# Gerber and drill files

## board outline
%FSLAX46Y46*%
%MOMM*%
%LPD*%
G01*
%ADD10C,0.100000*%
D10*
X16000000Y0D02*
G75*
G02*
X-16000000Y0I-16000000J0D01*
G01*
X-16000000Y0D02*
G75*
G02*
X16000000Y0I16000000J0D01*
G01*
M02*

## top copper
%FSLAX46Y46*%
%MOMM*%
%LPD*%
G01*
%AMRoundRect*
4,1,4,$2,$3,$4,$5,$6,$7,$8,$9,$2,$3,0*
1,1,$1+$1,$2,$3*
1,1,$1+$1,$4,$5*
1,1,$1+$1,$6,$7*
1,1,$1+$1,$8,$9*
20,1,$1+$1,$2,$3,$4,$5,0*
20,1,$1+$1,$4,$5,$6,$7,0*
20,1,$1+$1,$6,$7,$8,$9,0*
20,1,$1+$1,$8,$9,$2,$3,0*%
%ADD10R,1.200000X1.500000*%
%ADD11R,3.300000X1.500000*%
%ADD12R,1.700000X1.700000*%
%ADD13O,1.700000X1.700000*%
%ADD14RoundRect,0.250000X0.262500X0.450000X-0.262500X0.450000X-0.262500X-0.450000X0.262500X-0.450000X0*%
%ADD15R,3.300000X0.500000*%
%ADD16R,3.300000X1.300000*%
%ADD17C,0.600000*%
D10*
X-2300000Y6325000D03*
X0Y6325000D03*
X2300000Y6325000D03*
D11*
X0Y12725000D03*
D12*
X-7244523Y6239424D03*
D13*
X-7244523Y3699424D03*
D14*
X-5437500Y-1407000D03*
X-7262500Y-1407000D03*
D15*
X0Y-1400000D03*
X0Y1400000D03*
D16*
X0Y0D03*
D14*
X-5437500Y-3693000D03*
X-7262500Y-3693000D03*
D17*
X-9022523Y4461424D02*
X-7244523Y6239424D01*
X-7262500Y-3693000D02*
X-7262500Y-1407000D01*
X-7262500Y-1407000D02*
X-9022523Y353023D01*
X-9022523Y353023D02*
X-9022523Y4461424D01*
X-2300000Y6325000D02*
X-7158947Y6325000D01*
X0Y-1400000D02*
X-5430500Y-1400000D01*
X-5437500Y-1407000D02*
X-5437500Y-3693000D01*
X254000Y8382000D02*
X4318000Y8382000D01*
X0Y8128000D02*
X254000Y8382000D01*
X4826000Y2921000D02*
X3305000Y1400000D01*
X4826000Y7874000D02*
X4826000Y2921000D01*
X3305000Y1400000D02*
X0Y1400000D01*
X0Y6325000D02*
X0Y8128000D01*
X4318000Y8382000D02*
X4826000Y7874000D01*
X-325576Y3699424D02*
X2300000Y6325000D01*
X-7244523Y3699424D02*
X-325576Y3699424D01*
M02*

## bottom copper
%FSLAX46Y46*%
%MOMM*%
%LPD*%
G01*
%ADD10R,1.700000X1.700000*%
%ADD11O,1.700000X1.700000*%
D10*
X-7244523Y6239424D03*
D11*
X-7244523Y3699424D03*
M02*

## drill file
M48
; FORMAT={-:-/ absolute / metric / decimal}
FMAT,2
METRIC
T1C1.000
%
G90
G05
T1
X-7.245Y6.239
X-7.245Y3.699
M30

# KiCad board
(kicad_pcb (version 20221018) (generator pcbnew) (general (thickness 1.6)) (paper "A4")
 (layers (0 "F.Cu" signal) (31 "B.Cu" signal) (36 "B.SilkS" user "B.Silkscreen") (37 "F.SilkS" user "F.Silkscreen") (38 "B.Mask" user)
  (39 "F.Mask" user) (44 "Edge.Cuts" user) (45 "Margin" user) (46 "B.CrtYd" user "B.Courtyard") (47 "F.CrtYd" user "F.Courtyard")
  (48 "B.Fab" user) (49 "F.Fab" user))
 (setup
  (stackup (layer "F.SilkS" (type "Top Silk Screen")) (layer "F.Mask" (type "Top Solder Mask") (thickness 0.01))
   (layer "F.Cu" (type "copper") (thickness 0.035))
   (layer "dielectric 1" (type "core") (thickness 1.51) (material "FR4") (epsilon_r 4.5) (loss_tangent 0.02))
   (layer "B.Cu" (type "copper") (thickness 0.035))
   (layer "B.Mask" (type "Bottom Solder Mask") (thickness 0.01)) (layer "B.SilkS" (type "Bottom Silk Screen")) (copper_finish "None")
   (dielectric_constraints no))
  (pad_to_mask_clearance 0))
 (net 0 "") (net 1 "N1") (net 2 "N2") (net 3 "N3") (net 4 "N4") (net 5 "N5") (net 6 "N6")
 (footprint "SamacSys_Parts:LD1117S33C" (layer "F.Cu") (at 0 -9.525)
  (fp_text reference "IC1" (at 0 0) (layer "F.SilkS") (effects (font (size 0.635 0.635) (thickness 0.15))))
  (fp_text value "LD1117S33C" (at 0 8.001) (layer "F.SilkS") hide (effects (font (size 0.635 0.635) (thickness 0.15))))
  (pad "1" smd rect (at -2.3 3.2) (size 1.2 1.5) (layers "F.Cu" "F.Paste" "F.Mask") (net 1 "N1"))
  (pad "2" smd rect (at 0 3.2) (size 1.2 1.5) (layers "F.Cu" "F.Paste" "F.Mask") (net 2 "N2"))
  (pad "3" smd rect (at 2.3 3.2) (size 1.2 1.5) (layers "F.Cu" "F.Paste" "F.Mask") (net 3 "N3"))
  (pad "4" smd rect (at 0 -3.2 90) (size 1.5 3.3) (layers "F.Cu" "F.Paste" "F.Mask") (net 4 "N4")))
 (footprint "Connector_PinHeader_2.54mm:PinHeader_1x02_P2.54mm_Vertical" (layer "F.Cu") (at -7.244523 -6.239424)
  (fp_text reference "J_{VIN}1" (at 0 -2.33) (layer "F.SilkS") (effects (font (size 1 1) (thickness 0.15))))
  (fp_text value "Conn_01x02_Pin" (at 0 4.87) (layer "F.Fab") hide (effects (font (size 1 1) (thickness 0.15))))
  (pad "1" thru_hole rect (at 0 0) (size 1.7 1.7) (drill 1) (layers "*.Cu" "*.Mask") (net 1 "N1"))
  (pad "2" thru_hole oval (at 0 2.54) (size 1.7 1.7) (drill 1) (layers "*.Cu" "*.Mask") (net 3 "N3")))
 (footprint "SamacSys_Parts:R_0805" (layer "F.Cu") (at -6.35 1.397 90)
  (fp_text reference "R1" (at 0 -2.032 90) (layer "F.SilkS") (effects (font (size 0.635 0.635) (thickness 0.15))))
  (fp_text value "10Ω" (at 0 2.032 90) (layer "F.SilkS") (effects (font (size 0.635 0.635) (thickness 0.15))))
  (pad "1" smd roundrect (at -0.01 0.9125 180) (size 1.025 1.4) (layers "F.Cu" "F.Paste" "F.Mask") (roundrect_rratio 0.243902439)
   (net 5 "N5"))
  (pad "2" smd roundrect (at -0.01 -0.9125 180) (size 1.025 1.4) (layers "F.Cu" "F.Paste" "F.Mask") (roundrect_rratio 0.243902439)
   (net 1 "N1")))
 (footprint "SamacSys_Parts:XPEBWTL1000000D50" (layer "F.Cu") (at 0 0 90)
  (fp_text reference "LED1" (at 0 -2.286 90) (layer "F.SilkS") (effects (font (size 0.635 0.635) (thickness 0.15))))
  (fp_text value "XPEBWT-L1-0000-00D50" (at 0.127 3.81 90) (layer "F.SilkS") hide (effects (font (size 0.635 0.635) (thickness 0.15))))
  (pad "1" smd rect (at -1.4 0 90) (size 0.5 3.3) (layers "F.Cu" "F.Paste" "F.Mask") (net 5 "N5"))
  (pad "2" smd rect (at 1.4 0 90) (size 0.5 3.3) (layers "F.Cu" "F.Paste" "F.Mask") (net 2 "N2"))
  (pad "3" smd rect (at 0 0 90) (size 1.3 3.3) (layers "F.Cu" "F.Paste" "F.Mask") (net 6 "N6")))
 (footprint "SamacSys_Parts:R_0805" (layer "F.Cu") (at -6.35 3.683 90)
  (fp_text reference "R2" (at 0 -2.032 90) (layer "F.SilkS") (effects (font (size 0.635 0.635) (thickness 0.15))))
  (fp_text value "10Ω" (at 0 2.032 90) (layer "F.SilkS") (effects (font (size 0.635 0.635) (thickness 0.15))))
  (pad "1" smd roundrect (at -0.01 0.9125 180) (size 1.025 1.4) (layers "F.Cu" "F.Paste" "F.Mask") (roundrect_rratio 0.243902439)
   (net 5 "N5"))
  (pad "2" smd roundrect (at -0.01 -0.9125 180) (size 1.025 1.4) (layers "F.Cu" "F.Paste" "F.Mask") (roundrect_rratio 0.243902439)
   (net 1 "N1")))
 (gr_circle (center 0 0) (end 16 0) (stroke (width 0.1) (type default)) (fill none) (layer "Edge.Cuts"))
 (segment (start -9.022523 -4.461424) (end -7.244523 -6.239424) (width 0.6) (layer "F.Cu") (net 1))
 (segment (start -7.2625 3.693) (end -7.2625 1.407) (width 0.6) (layer "F.Cu") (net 1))
 (segment (start -7.2625 1.407) (end -9.022523 -0.353023) (width 0.6) (layer "F.Cu") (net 1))
 (segment (start -9.022523 -0.353023) (end -9.022523 -4.461424) (width 0.6) (layer "F.Cu") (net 1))
 (segment (start -2.3 -6.325) (end -7.158947 -6.325) (width 0.6) (layer "F.Cu") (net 1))
 (segment (start 0 1.4) (end -5.4305 1.4) (width 0.6) (layer "F.Cu") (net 5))
 (segment (start -5.4375 1.407) (end -5.4375 3.693) (width 0.6) (layer "F.Cu") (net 5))
 (segment (start 0.254 -8.382) (end 4.318 -8.382) (width 0.6) (layer "F.Cu") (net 2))
 (segment (start 0 -8.128) (end 0.254 -8.382) (width 0.6) (layer "F.Cu") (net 2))
 (segment (start 4.826 -2.921) (end 3.305 -1.4) (width 0.6) (layer "F.Cu") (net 2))
 (segment (start 4.826 -7.874) (end 4.826 -2.921) (width 0.6) (layer "F.Cu") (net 2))
 (segment (start 3.305 -1.4) (end 0 -1.4) (width 0.6) (layer "F.Cu") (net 2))
 (segment (start 0 -6.325) (end 0 -8.128) (width 0.6) (layer "F.Cu") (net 2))
 (segment (start 4.318 -8.382) (end 4.826 -7.874) (width 0.6) (layer "F.Cu") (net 2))
 (segment (start -0.325576 -3.699424) (end 2.3 -6.325) (width 0.6) (layer "F.Cu") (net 3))
 (segment (start -7.244523 -3.699424) (end -0.325576 -3.699424) (width 0.6) (layer "F.Cu") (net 3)))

